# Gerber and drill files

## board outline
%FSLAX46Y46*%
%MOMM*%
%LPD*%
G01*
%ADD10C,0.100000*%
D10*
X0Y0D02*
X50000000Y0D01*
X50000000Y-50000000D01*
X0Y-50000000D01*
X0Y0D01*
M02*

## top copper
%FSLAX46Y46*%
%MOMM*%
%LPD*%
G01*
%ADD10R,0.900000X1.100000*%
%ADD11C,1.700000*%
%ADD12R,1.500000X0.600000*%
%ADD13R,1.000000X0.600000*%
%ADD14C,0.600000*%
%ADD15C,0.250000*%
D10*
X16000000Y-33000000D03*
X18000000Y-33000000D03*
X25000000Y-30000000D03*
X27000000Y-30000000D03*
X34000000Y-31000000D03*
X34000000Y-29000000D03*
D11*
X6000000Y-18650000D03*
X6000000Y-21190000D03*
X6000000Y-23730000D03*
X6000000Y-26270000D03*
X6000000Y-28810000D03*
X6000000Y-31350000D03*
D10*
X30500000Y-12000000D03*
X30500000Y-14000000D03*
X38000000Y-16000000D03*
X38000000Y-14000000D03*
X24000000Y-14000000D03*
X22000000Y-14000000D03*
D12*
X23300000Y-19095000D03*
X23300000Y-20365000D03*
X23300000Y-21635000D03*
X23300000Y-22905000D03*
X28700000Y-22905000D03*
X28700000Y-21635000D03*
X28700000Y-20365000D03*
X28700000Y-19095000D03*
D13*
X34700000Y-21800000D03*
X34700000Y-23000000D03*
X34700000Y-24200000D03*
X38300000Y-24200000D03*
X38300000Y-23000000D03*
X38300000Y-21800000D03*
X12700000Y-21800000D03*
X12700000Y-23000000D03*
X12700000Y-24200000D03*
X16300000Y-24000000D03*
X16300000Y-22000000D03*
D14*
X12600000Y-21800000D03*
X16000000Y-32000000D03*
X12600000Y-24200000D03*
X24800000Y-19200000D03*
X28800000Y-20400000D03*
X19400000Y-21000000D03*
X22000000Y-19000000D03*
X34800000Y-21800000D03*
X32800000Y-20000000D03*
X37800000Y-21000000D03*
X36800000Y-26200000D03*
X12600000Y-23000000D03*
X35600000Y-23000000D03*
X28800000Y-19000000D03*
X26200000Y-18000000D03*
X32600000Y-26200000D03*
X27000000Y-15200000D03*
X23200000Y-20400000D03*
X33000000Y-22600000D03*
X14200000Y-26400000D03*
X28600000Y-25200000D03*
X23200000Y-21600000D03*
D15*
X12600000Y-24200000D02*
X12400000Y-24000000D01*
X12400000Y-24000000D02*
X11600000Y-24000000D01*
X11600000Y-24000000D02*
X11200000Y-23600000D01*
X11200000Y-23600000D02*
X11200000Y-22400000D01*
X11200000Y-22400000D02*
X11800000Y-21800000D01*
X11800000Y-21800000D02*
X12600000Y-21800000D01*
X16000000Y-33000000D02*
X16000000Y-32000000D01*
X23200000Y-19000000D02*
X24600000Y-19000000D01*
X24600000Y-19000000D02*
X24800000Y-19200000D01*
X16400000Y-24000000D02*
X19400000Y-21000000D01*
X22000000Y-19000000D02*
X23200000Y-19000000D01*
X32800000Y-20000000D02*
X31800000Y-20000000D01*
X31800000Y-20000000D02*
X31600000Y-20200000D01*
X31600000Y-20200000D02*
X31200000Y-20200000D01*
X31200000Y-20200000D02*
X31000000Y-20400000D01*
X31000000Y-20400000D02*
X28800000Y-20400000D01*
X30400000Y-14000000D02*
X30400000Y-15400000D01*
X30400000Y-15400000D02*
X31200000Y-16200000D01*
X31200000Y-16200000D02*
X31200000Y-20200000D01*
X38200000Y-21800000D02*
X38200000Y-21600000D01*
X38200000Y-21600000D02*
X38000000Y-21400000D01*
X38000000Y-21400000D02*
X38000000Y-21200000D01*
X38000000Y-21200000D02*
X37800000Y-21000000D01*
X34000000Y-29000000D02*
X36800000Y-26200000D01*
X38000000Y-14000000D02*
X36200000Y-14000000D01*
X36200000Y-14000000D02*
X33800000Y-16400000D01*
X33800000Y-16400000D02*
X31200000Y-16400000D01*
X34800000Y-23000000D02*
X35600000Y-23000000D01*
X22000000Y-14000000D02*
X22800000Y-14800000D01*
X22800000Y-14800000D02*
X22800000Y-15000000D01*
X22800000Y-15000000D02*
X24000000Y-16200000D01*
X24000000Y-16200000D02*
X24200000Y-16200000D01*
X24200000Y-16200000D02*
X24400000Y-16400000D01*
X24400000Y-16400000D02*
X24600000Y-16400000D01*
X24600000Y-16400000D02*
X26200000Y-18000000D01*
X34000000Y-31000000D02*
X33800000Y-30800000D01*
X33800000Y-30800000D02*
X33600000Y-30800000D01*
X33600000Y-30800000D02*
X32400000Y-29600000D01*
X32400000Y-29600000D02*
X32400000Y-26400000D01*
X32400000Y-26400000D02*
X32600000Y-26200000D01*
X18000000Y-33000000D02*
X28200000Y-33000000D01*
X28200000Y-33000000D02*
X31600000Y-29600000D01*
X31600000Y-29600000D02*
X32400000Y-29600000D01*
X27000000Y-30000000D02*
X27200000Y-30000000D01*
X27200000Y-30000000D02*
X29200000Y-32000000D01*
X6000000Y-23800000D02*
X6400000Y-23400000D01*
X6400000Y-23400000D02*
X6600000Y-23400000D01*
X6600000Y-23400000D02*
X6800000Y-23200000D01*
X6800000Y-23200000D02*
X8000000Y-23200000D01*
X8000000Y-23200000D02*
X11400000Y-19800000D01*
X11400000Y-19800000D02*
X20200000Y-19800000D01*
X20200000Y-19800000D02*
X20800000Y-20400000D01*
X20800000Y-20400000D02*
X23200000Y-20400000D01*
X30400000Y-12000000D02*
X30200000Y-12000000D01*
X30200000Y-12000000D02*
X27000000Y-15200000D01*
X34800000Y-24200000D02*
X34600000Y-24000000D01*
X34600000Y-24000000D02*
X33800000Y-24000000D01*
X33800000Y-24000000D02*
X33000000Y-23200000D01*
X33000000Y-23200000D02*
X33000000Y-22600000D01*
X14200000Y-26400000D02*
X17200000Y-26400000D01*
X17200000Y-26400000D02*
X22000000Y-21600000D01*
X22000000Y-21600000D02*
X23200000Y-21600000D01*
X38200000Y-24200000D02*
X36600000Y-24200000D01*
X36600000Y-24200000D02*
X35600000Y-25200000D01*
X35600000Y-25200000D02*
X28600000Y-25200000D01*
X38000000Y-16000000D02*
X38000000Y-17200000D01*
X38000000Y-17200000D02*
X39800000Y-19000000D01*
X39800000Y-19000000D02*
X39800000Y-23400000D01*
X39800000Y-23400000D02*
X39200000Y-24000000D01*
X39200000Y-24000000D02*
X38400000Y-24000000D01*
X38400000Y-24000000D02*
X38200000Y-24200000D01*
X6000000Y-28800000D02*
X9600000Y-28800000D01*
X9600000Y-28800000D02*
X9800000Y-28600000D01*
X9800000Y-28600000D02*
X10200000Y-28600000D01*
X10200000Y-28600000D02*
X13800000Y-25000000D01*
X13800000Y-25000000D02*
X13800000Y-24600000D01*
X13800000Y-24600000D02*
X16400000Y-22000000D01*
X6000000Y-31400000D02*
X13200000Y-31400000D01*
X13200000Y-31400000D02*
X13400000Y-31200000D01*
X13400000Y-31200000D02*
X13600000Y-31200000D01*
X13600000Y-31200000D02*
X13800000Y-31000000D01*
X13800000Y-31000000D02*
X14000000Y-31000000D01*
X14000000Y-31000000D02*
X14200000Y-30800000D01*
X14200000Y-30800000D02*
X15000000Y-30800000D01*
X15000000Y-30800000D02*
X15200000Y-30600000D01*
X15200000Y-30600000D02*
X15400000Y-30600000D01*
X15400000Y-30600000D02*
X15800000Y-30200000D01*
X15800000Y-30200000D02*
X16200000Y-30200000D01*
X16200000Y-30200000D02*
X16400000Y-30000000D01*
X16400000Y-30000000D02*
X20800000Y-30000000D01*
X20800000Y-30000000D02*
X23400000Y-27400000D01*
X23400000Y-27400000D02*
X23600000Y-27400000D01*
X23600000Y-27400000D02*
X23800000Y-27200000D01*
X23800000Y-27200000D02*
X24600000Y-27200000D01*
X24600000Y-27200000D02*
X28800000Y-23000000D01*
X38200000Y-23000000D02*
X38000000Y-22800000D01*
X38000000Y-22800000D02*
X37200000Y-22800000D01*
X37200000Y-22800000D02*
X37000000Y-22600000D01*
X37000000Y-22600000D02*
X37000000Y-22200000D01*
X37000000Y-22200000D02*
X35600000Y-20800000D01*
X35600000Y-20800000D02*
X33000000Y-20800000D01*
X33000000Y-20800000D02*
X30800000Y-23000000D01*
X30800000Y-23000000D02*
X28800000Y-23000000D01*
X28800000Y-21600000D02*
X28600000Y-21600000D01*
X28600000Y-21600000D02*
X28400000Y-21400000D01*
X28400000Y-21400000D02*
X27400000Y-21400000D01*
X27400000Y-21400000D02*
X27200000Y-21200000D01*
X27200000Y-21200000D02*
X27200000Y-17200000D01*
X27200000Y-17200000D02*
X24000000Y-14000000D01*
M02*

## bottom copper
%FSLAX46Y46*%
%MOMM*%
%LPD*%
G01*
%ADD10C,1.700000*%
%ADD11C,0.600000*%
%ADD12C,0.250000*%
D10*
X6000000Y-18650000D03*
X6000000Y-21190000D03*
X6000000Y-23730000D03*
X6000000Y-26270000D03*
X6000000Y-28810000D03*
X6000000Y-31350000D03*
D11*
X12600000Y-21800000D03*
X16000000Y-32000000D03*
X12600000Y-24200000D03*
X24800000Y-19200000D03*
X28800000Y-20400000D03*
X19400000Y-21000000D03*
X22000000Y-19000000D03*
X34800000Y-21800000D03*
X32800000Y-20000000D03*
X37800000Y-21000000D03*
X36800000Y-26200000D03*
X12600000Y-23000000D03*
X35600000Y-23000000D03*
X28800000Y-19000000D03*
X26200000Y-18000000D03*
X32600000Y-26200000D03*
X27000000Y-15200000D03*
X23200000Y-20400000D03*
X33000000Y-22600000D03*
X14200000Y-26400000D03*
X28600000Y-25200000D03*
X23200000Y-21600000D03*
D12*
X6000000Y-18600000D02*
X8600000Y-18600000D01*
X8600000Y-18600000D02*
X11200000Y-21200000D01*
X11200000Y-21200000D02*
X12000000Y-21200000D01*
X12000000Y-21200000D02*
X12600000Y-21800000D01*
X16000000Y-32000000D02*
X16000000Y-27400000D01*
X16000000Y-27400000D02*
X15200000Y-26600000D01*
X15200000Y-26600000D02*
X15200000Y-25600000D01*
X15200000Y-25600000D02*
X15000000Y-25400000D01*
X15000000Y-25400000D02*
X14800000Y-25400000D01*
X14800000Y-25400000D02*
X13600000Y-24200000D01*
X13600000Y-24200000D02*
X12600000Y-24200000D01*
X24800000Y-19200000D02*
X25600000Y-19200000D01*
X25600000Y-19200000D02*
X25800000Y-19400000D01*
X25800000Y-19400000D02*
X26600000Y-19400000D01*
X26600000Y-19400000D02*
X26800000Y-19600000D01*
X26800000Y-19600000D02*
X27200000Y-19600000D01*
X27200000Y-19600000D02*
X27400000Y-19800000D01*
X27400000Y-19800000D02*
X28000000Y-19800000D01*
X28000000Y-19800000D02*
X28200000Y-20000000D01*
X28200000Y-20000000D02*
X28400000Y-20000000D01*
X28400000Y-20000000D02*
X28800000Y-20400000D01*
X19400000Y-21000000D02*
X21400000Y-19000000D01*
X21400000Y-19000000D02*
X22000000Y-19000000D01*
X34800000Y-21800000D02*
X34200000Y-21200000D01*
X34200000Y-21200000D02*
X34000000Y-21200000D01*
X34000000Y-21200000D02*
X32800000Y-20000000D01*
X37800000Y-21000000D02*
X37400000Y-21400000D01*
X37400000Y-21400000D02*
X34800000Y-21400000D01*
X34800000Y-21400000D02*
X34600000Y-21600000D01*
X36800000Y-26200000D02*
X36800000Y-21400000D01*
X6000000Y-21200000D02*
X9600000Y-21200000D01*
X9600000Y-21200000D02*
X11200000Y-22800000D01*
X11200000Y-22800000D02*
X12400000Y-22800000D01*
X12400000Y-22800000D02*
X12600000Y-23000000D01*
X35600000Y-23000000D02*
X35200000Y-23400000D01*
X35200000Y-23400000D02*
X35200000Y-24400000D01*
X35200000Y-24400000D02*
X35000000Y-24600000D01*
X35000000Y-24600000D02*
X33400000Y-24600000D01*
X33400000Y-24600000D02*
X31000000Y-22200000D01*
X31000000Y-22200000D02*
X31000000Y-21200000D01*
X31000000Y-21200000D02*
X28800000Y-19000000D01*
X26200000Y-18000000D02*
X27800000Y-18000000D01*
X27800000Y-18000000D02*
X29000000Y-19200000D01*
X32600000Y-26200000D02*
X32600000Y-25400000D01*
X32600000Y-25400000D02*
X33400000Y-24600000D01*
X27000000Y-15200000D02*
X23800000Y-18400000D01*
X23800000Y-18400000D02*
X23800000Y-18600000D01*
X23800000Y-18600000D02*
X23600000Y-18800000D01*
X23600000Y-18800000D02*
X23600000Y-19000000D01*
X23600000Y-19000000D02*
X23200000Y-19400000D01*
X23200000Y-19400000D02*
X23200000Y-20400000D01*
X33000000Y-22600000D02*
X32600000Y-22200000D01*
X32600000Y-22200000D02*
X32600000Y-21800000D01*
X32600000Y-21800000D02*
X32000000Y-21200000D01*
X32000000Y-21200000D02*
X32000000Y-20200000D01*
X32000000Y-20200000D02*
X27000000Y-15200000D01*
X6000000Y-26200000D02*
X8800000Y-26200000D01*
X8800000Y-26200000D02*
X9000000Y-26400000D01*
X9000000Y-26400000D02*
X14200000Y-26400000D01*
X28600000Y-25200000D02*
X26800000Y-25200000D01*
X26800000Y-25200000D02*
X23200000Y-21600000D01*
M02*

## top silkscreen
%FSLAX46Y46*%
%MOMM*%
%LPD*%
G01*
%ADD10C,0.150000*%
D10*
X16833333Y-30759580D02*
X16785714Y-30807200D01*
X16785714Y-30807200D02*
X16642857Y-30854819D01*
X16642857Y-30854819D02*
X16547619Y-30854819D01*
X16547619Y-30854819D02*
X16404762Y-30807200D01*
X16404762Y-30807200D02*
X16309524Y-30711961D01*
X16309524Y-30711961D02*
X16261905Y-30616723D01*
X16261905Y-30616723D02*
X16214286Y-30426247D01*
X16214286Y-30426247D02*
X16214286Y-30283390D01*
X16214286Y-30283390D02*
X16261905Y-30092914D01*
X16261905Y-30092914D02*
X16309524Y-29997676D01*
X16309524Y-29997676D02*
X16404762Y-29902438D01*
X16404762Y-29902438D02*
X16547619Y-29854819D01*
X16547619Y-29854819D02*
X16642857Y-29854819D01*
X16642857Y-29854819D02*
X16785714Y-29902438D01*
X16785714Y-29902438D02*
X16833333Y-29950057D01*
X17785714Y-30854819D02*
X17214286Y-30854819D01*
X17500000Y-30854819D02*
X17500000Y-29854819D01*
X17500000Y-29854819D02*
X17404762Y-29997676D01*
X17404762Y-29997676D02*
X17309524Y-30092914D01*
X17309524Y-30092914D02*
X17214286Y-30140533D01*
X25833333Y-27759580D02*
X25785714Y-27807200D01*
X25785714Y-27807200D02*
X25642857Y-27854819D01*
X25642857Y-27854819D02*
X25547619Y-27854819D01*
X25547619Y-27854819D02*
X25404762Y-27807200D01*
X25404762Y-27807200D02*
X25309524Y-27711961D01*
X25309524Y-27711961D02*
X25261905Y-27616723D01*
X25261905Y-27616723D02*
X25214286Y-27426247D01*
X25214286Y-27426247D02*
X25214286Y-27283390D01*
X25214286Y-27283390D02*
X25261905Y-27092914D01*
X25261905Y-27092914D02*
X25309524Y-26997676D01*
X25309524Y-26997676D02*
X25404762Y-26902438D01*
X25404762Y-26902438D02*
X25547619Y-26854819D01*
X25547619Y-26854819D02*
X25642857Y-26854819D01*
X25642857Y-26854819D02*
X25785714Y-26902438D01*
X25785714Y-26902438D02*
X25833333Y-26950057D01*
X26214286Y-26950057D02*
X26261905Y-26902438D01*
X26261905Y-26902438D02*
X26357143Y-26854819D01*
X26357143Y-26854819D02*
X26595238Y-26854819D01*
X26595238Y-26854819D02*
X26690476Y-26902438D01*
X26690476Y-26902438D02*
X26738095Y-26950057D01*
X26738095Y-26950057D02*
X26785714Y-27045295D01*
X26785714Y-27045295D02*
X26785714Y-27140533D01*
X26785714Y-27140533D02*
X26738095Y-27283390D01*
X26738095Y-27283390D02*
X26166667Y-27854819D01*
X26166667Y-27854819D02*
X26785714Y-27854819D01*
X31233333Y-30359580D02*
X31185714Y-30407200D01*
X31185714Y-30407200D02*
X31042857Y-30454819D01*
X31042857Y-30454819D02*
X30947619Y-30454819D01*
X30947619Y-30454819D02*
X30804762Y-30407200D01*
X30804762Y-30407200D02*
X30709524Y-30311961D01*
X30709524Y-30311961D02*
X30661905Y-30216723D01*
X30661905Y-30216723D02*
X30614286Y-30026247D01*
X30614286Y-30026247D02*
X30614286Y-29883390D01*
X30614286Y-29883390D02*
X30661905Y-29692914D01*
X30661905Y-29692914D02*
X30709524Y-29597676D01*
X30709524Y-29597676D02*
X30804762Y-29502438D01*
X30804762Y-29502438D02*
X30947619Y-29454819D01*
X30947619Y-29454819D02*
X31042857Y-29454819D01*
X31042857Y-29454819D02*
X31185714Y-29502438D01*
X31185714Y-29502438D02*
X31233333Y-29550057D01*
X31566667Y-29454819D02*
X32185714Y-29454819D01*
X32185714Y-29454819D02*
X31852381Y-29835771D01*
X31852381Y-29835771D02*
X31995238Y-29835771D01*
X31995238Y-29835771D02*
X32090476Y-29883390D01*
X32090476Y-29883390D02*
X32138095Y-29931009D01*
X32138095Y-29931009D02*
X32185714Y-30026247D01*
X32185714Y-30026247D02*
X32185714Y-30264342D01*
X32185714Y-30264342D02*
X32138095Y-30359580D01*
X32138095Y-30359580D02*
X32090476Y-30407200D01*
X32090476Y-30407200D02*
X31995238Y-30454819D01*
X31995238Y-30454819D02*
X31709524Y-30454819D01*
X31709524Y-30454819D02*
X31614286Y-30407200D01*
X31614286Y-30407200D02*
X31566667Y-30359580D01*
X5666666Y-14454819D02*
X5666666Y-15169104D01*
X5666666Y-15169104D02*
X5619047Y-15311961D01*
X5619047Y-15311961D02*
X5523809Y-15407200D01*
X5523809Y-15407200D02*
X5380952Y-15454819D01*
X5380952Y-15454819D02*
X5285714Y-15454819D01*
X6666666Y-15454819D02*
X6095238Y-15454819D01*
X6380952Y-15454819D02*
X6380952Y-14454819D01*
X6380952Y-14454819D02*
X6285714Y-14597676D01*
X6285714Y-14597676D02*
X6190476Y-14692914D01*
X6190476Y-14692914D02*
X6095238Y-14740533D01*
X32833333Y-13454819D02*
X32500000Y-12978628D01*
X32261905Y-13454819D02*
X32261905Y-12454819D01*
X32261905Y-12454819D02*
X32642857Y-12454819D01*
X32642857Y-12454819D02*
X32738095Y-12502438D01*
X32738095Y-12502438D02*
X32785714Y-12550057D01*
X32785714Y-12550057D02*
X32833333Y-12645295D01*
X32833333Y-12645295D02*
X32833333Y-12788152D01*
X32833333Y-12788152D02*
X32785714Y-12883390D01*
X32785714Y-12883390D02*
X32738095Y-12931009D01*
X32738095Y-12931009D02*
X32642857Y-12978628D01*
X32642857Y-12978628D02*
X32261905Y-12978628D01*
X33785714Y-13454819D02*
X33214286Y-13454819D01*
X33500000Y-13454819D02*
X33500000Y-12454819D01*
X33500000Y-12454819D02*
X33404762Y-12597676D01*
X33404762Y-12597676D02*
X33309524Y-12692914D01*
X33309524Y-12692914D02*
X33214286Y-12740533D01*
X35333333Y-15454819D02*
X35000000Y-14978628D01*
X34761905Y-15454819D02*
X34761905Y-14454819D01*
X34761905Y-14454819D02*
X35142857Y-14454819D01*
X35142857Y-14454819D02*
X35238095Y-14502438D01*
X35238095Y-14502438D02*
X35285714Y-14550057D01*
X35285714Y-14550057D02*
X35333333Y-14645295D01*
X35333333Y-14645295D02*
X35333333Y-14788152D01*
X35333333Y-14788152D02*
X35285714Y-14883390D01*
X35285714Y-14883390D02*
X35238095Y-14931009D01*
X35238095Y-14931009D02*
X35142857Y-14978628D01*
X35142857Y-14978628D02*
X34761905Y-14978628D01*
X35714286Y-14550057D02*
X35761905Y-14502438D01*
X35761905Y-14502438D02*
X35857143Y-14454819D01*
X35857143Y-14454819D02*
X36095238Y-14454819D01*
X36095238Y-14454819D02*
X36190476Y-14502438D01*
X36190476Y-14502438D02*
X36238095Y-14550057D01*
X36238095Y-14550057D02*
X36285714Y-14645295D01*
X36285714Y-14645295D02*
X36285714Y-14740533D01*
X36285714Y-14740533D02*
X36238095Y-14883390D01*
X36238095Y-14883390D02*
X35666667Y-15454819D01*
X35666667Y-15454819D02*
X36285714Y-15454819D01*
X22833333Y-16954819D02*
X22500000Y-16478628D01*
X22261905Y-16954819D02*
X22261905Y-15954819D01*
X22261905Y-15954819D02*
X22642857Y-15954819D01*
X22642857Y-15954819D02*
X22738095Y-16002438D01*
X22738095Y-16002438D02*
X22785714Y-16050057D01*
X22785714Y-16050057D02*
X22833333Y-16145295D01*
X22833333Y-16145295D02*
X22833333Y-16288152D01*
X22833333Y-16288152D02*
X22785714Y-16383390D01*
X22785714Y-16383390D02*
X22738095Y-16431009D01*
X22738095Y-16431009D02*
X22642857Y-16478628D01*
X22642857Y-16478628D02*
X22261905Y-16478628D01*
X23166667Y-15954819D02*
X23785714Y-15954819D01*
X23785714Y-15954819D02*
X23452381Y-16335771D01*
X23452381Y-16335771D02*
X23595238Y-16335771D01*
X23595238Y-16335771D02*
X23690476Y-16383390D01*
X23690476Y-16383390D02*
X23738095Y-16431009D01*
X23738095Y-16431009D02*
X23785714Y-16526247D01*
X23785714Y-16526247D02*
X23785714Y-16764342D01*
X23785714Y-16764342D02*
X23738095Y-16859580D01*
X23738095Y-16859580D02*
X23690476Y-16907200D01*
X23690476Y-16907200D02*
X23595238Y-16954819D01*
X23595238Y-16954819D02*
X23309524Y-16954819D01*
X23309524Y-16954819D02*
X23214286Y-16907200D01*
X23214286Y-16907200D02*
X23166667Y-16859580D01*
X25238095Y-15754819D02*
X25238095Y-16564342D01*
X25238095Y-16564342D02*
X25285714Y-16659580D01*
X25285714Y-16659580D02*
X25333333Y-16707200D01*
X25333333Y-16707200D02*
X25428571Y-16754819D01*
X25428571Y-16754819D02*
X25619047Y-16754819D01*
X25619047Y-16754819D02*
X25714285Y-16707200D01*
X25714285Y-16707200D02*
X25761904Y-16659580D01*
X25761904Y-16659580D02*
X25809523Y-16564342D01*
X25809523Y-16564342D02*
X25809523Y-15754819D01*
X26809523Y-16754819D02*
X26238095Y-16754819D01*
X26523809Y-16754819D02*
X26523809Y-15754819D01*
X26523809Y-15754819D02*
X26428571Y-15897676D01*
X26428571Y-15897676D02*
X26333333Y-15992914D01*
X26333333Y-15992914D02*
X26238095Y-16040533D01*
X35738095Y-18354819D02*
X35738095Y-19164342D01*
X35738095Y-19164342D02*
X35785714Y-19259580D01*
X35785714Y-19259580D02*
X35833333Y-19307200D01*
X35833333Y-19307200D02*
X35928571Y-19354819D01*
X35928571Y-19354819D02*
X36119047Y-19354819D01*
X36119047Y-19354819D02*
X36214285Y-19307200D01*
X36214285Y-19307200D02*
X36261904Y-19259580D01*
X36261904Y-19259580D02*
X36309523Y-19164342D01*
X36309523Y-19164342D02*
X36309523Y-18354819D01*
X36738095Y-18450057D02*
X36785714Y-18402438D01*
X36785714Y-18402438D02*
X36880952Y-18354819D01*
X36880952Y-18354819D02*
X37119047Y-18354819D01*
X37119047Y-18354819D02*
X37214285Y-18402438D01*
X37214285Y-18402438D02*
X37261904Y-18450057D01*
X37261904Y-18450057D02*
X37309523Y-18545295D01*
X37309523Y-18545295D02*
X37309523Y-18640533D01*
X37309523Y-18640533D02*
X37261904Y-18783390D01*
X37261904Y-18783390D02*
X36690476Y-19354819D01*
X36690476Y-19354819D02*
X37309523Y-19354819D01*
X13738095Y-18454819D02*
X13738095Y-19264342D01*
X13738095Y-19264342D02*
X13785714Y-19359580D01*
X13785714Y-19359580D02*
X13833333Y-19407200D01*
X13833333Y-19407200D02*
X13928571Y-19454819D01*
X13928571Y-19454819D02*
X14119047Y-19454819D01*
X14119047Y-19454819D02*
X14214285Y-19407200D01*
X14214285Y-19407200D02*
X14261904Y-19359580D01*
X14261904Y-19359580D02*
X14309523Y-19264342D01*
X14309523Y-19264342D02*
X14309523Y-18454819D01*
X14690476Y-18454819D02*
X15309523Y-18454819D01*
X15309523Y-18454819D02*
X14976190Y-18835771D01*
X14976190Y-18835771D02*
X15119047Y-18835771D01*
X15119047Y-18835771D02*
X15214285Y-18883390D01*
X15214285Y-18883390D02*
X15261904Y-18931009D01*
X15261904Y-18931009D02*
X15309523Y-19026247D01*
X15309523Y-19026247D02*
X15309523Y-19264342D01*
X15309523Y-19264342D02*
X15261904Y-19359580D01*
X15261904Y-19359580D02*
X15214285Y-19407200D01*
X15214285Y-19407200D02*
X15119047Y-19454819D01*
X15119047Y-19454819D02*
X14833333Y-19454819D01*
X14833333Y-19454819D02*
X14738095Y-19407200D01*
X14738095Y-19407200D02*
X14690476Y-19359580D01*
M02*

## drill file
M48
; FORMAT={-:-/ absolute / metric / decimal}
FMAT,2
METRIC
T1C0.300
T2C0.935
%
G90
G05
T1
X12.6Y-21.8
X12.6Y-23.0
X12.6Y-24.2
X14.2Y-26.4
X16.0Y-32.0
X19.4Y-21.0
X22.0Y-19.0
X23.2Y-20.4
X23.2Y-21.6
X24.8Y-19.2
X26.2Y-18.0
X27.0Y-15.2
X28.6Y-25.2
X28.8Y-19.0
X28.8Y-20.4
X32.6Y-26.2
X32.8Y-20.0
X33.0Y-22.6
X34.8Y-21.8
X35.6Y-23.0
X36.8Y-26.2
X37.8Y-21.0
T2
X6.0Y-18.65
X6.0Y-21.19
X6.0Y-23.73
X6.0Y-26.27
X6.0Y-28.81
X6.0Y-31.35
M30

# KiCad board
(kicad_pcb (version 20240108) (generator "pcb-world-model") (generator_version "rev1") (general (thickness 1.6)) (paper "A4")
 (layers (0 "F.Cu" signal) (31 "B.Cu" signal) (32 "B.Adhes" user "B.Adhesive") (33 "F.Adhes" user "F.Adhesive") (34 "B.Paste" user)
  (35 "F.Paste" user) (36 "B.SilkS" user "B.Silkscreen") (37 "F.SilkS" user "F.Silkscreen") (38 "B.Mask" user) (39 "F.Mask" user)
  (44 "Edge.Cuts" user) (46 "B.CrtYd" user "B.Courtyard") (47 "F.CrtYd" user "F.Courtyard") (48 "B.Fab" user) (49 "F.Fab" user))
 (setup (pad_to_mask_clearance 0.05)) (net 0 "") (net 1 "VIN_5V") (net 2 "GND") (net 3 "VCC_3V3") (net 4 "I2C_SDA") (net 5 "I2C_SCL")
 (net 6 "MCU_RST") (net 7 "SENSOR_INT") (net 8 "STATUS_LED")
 (gr_rect (start 0.0 0.0) (end 50.0000 50.0000) (stroke (width 0.1) (type default)) (fill none) (layer "Edge.Cuts"))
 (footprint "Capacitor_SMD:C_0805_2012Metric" (layer "F.Cu") (at 17.0000 33.0000 0)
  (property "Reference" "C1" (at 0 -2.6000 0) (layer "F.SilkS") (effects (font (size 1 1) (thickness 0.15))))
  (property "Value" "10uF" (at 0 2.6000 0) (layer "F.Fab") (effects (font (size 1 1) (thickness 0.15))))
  (pad "1" smd rect (at -1.0000 0.0000) (size 0.9000 1.1000) (layers "F.Cu" "F.Paste" "F.Mask") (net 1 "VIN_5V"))
  (pad "2" smd rect (at 1.0000 0.0000) (size 0.9000 1.1000) (layers "F.Cu" "F.Paste" "F.Mask") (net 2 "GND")))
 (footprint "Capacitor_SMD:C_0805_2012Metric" (layer "F.Cu") (at 26.0000 30.0000 0)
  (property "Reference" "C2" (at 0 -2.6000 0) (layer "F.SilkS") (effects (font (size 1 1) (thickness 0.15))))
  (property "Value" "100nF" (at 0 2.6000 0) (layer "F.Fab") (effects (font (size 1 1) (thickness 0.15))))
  (pad "1" smd rect (at -1.0000 0.0000) (size 0.9000 1.1000) (layers "F.Cu" "F.Paste" "F.Mask") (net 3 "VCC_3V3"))
  (pad "2" smd rect (at 1.0000 0.0000) (size 0.9000 1.1000) (layers "F.Cu" "F.Paste" "F.Mask") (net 2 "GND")))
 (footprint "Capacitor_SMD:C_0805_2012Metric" (layer "F.Cu") (at 34.0000 30.0000 90)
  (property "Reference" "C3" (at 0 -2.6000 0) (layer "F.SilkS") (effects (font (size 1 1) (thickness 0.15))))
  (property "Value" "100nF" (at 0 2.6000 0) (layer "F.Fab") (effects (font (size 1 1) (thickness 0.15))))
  (pad "1" smd rect (at -1.0000 0.0000) (size 0.9000 1.1000) (layers "F.Cu" "F.Paste" "F.Mask") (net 3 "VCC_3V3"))
  (pad "2" smd rect (at 1.0000 0.0000) (size 0.9000 1.1000) (layers "F.Cu" "F.Paste" "F.Mask") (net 2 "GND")))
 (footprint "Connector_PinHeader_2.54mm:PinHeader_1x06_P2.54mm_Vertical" (layer "F.Cu") (at 6.0000 25.0000 0) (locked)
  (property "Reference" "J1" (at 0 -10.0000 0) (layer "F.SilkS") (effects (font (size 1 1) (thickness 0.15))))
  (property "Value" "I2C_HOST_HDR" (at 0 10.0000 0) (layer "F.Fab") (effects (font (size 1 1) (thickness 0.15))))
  (pad "1" thru_hole circle (at 0.0000 -6.3500) (size 1.7000 1.7000) (drill 0.9350) (layers "*.Cu" "*.Mask") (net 1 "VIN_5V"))
  (pad "2" thru_hole circle (at 0.0000 -3.8100) (size 1.7000 1.7000) (drill 0.9350) (layers "*.Cu" "*.Mask") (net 2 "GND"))
  (pad "3" thru_hole circle (at 0.0000 -1.2700) (size 1.7000 1.7000) (drill 0.9350) (layers "*.Cu" "*.Mask") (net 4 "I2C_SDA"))
  (pad "4" thru_hole circle (at 0.0000 1.2700) (size 1.7000 1.7000) (drill 0.9350) (layers "*.Cu" "*.Mask") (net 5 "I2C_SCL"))
  (pad "5" thru_hole circle (at 0.0000 3.8100) (size 1.7000 1.7000) (drill 0.9350) (layers "*.Cu" "*.Mask") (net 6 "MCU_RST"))
  (pad "6" thru_hole circle (at 0.0000 6.3500) (size 1.7000 1.7000) (drill 0.9350) (layers "*.Cu" "*.Mask") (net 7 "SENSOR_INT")))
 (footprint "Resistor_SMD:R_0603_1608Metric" (layer "F.Cu") (at 30.5000 13.0000 270)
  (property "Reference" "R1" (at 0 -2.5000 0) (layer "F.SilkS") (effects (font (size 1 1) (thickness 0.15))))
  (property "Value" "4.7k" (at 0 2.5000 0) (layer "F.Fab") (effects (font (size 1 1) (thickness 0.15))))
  (pad "1" smd rect (at -1.0000 0.0000) (size 0.9000 1.1000) (layers "F.Cu" "F.Paste" "F.Mask") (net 3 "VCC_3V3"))
  (pad "2" smd rect (at 1.0000 0.0000) (size 0.9000 1.1000) (layers "F.Cu" "F.Paste" "F.Mask") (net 4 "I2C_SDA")))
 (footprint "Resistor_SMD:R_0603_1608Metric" (layer "F.Cu") (at 38.0000 15.0000 90)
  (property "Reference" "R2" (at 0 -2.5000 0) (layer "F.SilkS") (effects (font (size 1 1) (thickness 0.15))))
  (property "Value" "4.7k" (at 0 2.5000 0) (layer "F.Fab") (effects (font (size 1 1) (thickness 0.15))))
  (pad "1" smd rect (at -1.0000 0.0000) (size 0.9000 1.1000) (layers "F.Cu" "F.Paste" "F.Mask") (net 3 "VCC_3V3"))
  (pad "2" smd rect (at 1.0000 0.0000) (size 0.9000 1.1000) (layers "F.Cu" "F.Paste" "F.Mask") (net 5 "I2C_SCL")))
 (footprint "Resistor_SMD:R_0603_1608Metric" (layer "F.Cu") (at 23.0000 14.0000 180)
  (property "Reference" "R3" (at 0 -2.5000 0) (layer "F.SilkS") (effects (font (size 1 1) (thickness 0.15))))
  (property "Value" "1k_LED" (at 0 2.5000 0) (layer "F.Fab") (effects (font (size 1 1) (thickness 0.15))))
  (pad "1" smd rect (at -1.0000 0.0000) (size 0.9000 1.1000) (layers "F.Cu" "F.Paste" "F.Mask") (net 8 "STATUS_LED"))
  (pad "2" smd rect (at 1.0000 0.0000) (size 0.9000 1.1000) (layers "F.Cu" "F.Paste" "F.Mask") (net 2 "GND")))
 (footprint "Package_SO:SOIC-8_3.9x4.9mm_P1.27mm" (layer "F.Cu") (at 26.0000 21.0000 0)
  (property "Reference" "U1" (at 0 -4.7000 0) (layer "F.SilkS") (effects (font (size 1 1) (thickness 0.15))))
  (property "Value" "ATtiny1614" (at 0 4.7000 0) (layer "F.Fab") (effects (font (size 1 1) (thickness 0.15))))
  (pad "1" smd rect (at -2.7000 -1.9050) (size 1.5000 0.6000) (layers "F.Cu" "F.Paste" "F.Mask") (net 3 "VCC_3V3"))
  (pad "2" smd rect (at -2.7000 -0.6350) (size 1.5000 0.6000) (layers "F.Cu" "F.Paste" "F.Mask") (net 4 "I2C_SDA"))
  (pad "3" smd rect (at -2.7000 0.6350) (size 1.5000 0.6000) (layers "F.Cu" "F.Paste" "F.Mask") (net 5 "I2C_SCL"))
  (pad "4" smd rect (at -2.7000 1.9050) (size 1.5000 0.6000) (layers "F.Cu" "F.Paste" "F.Mask") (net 6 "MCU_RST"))
  (pad "5" smd rect (at 2.7000 1.9050) (size 1.5000 0.6000) (layers "F.Cu" "F.Paste" "F.Mask") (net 7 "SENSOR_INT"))
  (pad "6" smd rect (at 2.7000 0.6350) (size 1.5000 0.6000) (layers "F.Cu" "F.Paste" "F.Mask") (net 8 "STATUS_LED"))
  (pad "7" smd rect (at 2.7000 -0.6350) (size 1.5000 0.6000) (layers "F.Cu" "F.Paste" "F.Mask") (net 3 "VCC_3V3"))
  (pad "8" smd rect (at 2.7000 -1.9050) (size 1.5000 0.6000) (layers "F.Cu" "F.Paste" "F.Mask") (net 2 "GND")))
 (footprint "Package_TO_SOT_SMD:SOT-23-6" (layer "F.Cu") (at 36.5000 23.0000 0)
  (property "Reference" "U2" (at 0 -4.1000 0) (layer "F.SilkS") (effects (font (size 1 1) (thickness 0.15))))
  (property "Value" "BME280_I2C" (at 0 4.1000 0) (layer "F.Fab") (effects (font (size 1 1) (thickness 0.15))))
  (pad "1" smd rect (at -1.8000 -1.2000) (size 1.0000 0.6000) (layers "F.Cu" "F.Paste" "F.Mask") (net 3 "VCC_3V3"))
  (pad "2" smd rect (at -1.8000 0.0000) (size 1.0000 0.6000) (layers "F.Cu" "F.Paste" "F.Mask") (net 2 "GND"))
  (pad "3" smd rect (at -1.8000 1.2000) (size 1.0000 0.6000) (layers "F.Cu" "F.Paste" "F.Mask") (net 4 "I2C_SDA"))
  (pad "4" smd rect (at 1.8000 1.2000) (size 1.0000 0.6000) (layers "F.Cu" "F.Paste" "F.Mask") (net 5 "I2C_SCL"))
  (pad "5" smd rect (at 1.8000 0.0000) (size 1.0000 0.6000) (layers "F.Cu" "F.Paste" "F.Mask") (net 7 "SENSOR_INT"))
  (pad "6" smd rect (at 1.8000 -1.2000) (size 1.0000 0.6000) (layers "F.Cu" "F.Paste" "F.Mask") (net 3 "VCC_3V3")))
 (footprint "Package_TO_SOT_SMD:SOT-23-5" (layer "F.Cu") (at 14.5000 23.0000 0)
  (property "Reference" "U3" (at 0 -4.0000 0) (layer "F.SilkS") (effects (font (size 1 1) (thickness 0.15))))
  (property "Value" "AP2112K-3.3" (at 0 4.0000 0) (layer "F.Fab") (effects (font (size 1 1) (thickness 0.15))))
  (pad "1" smd rect (at -1.8000 -1.2000) (size 1.0000 0.6000) (layers "F.Cu" "F.Paste" "F.Mask") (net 1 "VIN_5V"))
  (pad "2" smd rect (at -1.8000 0.0000) (size 1.0000 0.6000) (layers "F.Cu" "F.Paste" "F.Mask") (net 2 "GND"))
  (pad "3" smd rect (at -1.8000 1.2000) (size 1.0000 0.6000) (layers "F.Cu" "F.Paste" "F.Mask") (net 1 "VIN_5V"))
  (pad "4" smd rect (at 1.8000 1.0000) (size 1.0000 0.6000) (layers "F.Cu" "F.Paste" "F.Mask") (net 3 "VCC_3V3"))
  (pad "5" smd rect (at 1.8000 -1.0000) (size 1.0000 0.6000) (layers "F.Cu" "F.Paste" "F.Mask") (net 6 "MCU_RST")))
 (segment (start 6.0000 18.6000) (end 8.6000 18.6000) (width 0.2500) (layer "B.Cu") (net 1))
 (segment (start 8.6000 18.6000) (end 11.2000 21.2000) (width 0.2500) (layer "B.Cu") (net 1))
 (segment (start 11.2000 21.2000) (end 12.0000 21.2000) (width 0.2500) (layer "B.Cu") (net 1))
 (segment (start 12.0000 21.2000) (end 12.6000 21.8000) (width 0.2500) (layer "B.Cu") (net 1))
 (segment (start 12.6000 24.2000) (end 12.4000 24.0000) (width 0.2500) (layer "F.Cu") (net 1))
 (segment (start 12.4000 24.0000) (end 11.6000 24.0000) (width 0.2500) (layer "F.Cu") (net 1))
 (segment (start 11.6000 24.0000) (end 11.2000 23.6000) (width 0.2500) (layer "F.Cu") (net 1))
 (segment (start 11.2000 23.6000) (end 11.2000 22.4000) (width 0.2500) (layer "F.Cu") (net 1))
 (segment (start 11.2000 22.4000) (end 11.8000 21.8000) (width 0.2500) (layer "F.Cu") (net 1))
 (segment (start 11.8000 21.8000) (end 12.6000 21.8000) (width 0.2500) (layer "F.Cu") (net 1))
 (segment (start 16.0000 33.0000) (end 16.0000 32.0000) (width 0.2500) (layer "F.Cu") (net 1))
 (segment (start 16.0000 32.0000) (end 16.0000 27.4000) (width 0.2500) (layer "B.Cu") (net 1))
 (segment (start 16.0000 27.4000) (end 15.2000 26.6000) (width 0.2500) (layer "B.Cu") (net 1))
 (segment (start 15.2000 26.6000) (end 15.2000 25.6000) (width 0.2500) (layer "B.Cu") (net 1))
 (segment (start 15.2000 25.6000) (end 15.0000 25.4000) (width 0.2500) (layer "B.Cu") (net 1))
 (segment (start 15.0000 25.4000) (end 14.8000 25.4000) (width 0.2500) (layer "B.Cu") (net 1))
 (segment (start 14.8000 25.4000) (end 13.6000 24.2000) (width 0.2500) (layer "B.Cu") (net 1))
 (segment (start 13.6000 24.2000) (end 12.6000 24.2000) (width 0.2500) (layer "B.Cu") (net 1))
 (segment (start 23.2000 19.0000) (end 24.6000 19.0000) (width 0.2500) (layer "F.Cu") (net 3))
 (segment (start 24.6000 19.0000) (end 24.8000 19.2000) (width 0.2500) (layer "F.Cu") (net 3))
 (segment (start 24.8000 19.2000) (end 25.6000 19.2000) (width 0.2500) (layer "B.Cu") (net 3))
 (segment (start 25.6000 19.2000) (end 25.8000 19.4000) (width 0.2500) (layer "B.Cu") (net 3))
 (segment (start 25.8000 19.4000) (end 26.6000 19.4000) (width 0.2500) (layer "B.Cu") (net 3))
 (segment (start 26.6000 19.4000) (end 26.8000 19.6000) (width 0.2500) (layer "B.Cu") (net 3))
 (segment (start 26.8000 19.6000) (end 27.2000 19.6000) (width 0.2500) (layer "B.Cu") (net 3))
 (segment (start 27.2000 19.6000) (end 27.4000 19.8000) (width 0.2500) (layer "B.Cu") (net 3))
 (segment (start 27.4000 19.8000) (end 28.0000 19.8000) (width 0.2500) (layer "B.Cu") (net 3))
 (segment (start 28.0000 19.8000) (end 28.2000 20.0000) (width 0.2500) (layer "B.Cu") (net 3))
 (segment (start 28.2000 20.0000) (end 28.4000 20.0000) (width 0.2500) (layer "B.Cu") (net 3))
 (segment (start 28.4000 20.0000) (end 28.8000 20.4000) (width 0.2500) (layer "B.Cu") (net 3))
 (segment (start 16.4000 24.0000) (end 19.4000 21.0000) (width 0.2500) (layer "F.Cu") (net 3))
 (segment (start 19.4000 21.0000) (end 21.4000 19.0000) (width 0.2500) (layer "B.Cu") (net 3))
 (segment (start 21.4000 19.0000) (end 22.0000 19.0000) (width 0.2500) (layer "B.Cu") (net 3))
 (segment (start 22.0000 19.0000) (end 23.2000 19.0000) (width 0.2500) (layer "F.Cu") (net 3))
 (segment (start 34.8000 21.8000) (end 34.2000 21.2000) (width 0.2500) (layer "B.Cu") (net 3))
 (segment (start 34.2000 21.2000) (end 34.0000 21.2000) (width 0.2500) (layer "B.Cu") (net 3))
 (segment (start 34.0000 21.2000) (end 32.8000 20.0000) (width 0.2500) (layer "B.Cu") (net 3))
 (segment (start 32.8000 20.0000) (end 31.8000 20.0000) (width 0.2500) (layer "F.Cu") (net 3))
 (segment (start 31.8000 20.0000) (end 31.6000 20.2000) (width 0.2500) (layer "F.Cu") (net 3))
 (segment (start 31.6000 20.2000) (end 31.2000 20.2000) (width 0.2500) (layer "F.Cu") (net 3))
 (segment (start 31.2000 20.2000) (end 31.0000 20.4000) (width 0.2500) (layer "F.Cu") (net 3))
 (segment (start 31.0000 20.4000) (end 28.8000 20.4000) (width 0.2500) (layer "F.Cu") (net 3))
 (segment (start 30.4000 14.0000) (end 30.4000 15.4000) (width 0.2500) (layer "F.Cu") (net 3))
 (segment (start 30.4000 15.4000) (end 31.2000 16.2000) (width 0.2500) (layer "F.Cu") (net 3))
 (segment (start 31.2000 16.2000) (end 31.2000 20.2000) (width 0.2500) (layer "F.Cu") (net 3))
 (segment (start 38.2000 21.8000) (end 38.2000 21.6000) (width 0.2500) (layer "F.Cu") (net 3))
 (segment (start 38.2000 21.6000) (end 38.0000 21.4000) (width 0.2500) (layer "F.Cu") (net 3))
 (segment (start 38.0000 21.4000) (end 38.0000 21.2000) (width 0.2500) (layer "F.Cu") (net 3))
 (segment (start 38.0000 21.2000) (end 37.8000 21.0000) (width 0.2500) (layer "F.Cu") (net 3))
 (segment (start 37.8000 21.0000) (end 37.4000 21.4000) (width 0.2500) (layer "B.Cu") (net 3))
 (segment (start 37.4000 21.4000) (end 34.8000 21.4000) (width 0.2500) (layer "B.Cu") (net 3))
 (segment (start 34.8000 21.4000) (end 34.6000 21.6000) (width 0.2500) (layer "B.Cu") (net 3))
 (segment (start 34.0000 29.0000) (end 36.8000 26.2000) (width 0.2500) (layer "F.Cu") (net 3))
 (segment (start 36.8000 26.2000) (end 36.8000 21.4000) (width 0.2500) (layer "B.Cu") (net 3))
 (segment (start 38.0000 14.0000) (end 36.2000 14.0000) (width 0.2500) (layer "F.Cu") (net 3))
 (segment (start 36.2000 14.0000) (end 33.8000 16.4000) (width 0.2500) (layer "F.Cu") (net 3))
 (segment (start 33.8000 16.4000) (end 31.2000 16.4000) (width 0.2500) (layer "F.Cu") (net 3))
 (segment (start 6.0000 21.2000) (end 9.6000 21.2000) (width 0.2500) (layer "B.Cu") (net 2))
 (segment (start 9.6000 21.2000) (end 11.2000 22.8000) (width 0.2500) (layer "B.Cu") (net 2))
 (segment (start 11.2000 22.8000) (end 12.4000 22.8000) (width 0.2500) (layer "B.Cu") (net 2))
 (segment (start 12.4000 22.8000) (end 12.6000 23.0000) (width 0.2500) (layer "B.Cu") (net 2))
 (segment (start 34.8000 23.0000) (end 35.6000 23.0000) (width 0.2500) (layer "F.Cu") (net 2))
 (segment (start 35.6000 23.0000) (end 35.2000 23.4000) (width 0.2500) (layer "B.Cu") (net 2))
 (segment (start 35.2000 23.4000) (end 35.2000 24.4000) (width 0.2500) (layer "B.Cu") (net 2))
 (segment (start 35.2000 24.4000) (end 35.0000 24.6000) (width 0.2500) (layer "B.Cu") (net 2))
 (segment (start 35.0000 24.6000) (end 33.4000 24.6000) (width 0.2500) (layer "B.Cu") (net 2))
 (segment (start 33.4000 24.6000) (end 31.0000 22.2000) (width 0.2500) (layer "B.Cu") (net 2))
 (segment (start 31.0000 22.2000) (end 31.0000 21.2000) (width 0.2500) (layer "B.Cu") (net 2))
 (segment (start 31.0000 21.2000) (end 28.8000 19.0000) (width 0.2500) (layer "B.Cu") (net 2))
 (segment (start 22.0000 14.0000) (end 22.8000 14.8000) (width 0.2500) (layer "F.Cu") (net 2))
 (segment (start 22.8000 14.8000) (end 22.8000 15.0000) (width 0.2500) (layer "F.Cu") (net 2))
 (segment (start 22.8000 15.0000) (end 24.0000 16.2000) (width 0.2500) (layer "F.Cu") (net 2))
 (segment (start 24.0000 16.2000) (end 24.2000 16.2000) (width 0.2500) (layer "F.Cu") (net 2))
 (segment (start 24.2000 16.2000) (end 24.4000 16.4000) (width 0.2500) (layer "F.Cu") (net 2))
 (segment (start 24.4000 16.4000) (end 24.6000 16.4000) (width 0.2500) (layer "F.Cu") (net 2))
 (segment (start 24.6000 16.4000) (end 26.2000 18.0000) (width 0.2500) (layer "F.Cu") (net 2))
 (segment (start 26.2000 18.0000) (end 27.8000 18.0000) (width 0.2500) (layer "B.Cu") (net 2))
 (segment (start 27.8000 18.0000) (end 29.0000 19.2000) (width 0.2500) (layer "B.Cu") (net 2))
 (segment (start 34.0000 31.0000) (end 33.8000 30.8000) (width 0.2500) (layer "F.Cu") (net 2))
 (segment (start 33.8000 30.8000) (end 33.6000 30.8000) (width 0.2500) (layer "F.Cu") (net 2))
 (segment (start 33.6000 30.8000) (end 32.4000 29.6000) (width 0.2500) (layer "F.Cu") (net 2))
 (segment (start 32.4000 29.6000) (end 32.4000 26.4000) (width 0.2500) (layer "F.Cu") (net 2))
 (segment (start 32.4000 26.4000) (end 32.6000 26.2000) (width 0.2500) (layer "F.Cu") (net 2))
 (segment (start 32.6000 26.2000) (end 32.6000 25.4000) (width 0.2500) (layer "B.Cu") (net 2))
 (segment (start 32.6000 25.4000) (end 33.4000 24.6000) (width 0.2500) (layer "B.Cu") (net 2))
 (segment (start 18.0000 33.0000) (end 28.2000 33.0000) (width 0.2500) (layer "F.Cu") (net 2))
 (segment (start 28.2000 33.0000) (end 31.6000 29.6000) (width 0.2500) (layer "F.Cu") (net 2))
 (segment (start 31.6000 29.6000) (end 32.4000 29.6000) (width 0.2500) (layer "F.Cu") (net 2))
 (segment (start 27.0000 30.0000) (end 27.2000 30.0000) (width 0.2500) (layer "F.Cu") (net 2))
 (segment (start 27.2000 30.0000) (end 29.2000 32.0000) (width 0.2500) (layer "F.Cu") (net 2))
 (segment (start 6.0000 23.8000) (end 6.4000 23.4000) (width 0.2500) (layer "F.Cu") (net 4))
 (segment (start 6.4000 23.4000) (end 6.6000 23.4000) (width 0.2500) (layer "F.Cu") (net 4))
 (segment (start 6.6000 23.4000) (end 6.8000 23.2000) (width 0.2500) (layer "F.Cu") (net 4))
 (segment (start 6.8000 23.2000) (end 8.0000 23.2000) (width 0.2500) (layer "F.Cu") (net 4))
 (segment (start 8.0000 23.2000) (end 11.4000 19.8000) (width 0.2500) (layer "F.Cu") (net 4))
 (segment (start 11.4000 19.8000) (end 20.2000 19.8000) (width 0.2500) (layer "F.Cu") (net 4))
 (segment (start 20.2000 19.8000) (end 20.8000 20.4000) (width 0.2500) (layer "F.Cu") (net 4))
 (segment (start 20.8000 20.4000) (end 23.2000 20.4000) (width 0.2500) (layer "F.Cu") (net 4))
 (segment (start 30.4000 12.0000) (end 30.2000 12.0000) (width 0.2500) (layer "F.Cu") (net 4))
 (segment (start 30.2000 12.0000) (end 27.0000 15.2000) (width 0.2500) (layer "F.Cu") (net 4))
 (segment (start 27.0000 15.2000) (end 23.8000 18.4000) (width 0.2500) (layer "B.Cu") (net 4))
 (segment (start 23.8000 18.4000) (end 23.8000 18.6000) (width 0.2500) (layer "B.Cu") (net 4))
 (segment (start 23.8000 18.6000) (end 23.6000 18.8000) (width 0.2500) (layer "B.Cu") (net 4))
 (segment (start 23.6000 18.8000) (end 23.6000 19.0000) (width 0.2500) (layer "B.Cu") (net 4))
 (segment (start 23.6000 19.0000) (end 23.2000 19.4000) (width 0.2500) (layer "B.Cu") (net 4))
 (segment (start 23.2000 19.4000) (end 23.2000 20.4000) (width 0.2500) (layer "B.Cu") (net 4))
 (segment (start 34.8000 24.2000) (end 34.6000 24.0000) (width 0.2500) (layer "F.Cu") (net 4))
 (segment (start 34.6000 24.0000) (end 33.8000 24.0000) (width 0.2500) (layer "F.Cu") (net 4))
 (segment (start 33.8000 24.0000) (end 33.0000 23.2000) (width 0.2500) (layer "F.Cu") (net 4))
 (segment (start 33.0000 23.2000) (end 33.0000 22.6000) (width 0.2500) (layer "F.Cu") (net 4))
 (segment (start 33.0000 22.6000) (end 32.6000 22.2000) (width 0.2500) (layer "B.Cu") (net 4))
 (segment (start 32.6000 22.2000) (end 32.6000 21.8000) (width 0.2500) (layer "B.Cu") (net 4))
 (segment (start 32.6000 21.8000) (end 32.0000 21.2000) (width 0.2500) (layer "B.Cu") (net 4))
 (segment (start 32.0000 21.2000) (end 32.0000 20.2000) (width 0.2500) (layer "B.Cu") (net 4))
 (segment (start 32.0000 20.2000) (end 27.0000 15.2000) (width 0.2500) (layer "B.Cu") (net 4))
 (segment (start 6.0000 26.2000) (end 8.8000 26.2000) (width 0.2500) (layer "B.Cu") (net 5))
 (segment (start 8.8000 26.2000) (end 9.0000 26.4000) (width 0.2500) (layer "B.Cu") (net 5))
 (segment (start 9.0000 26.4000) (end 14.2000 26.4000) (width 0.2500) (layer "B.Cu") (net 5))
 (segment (start 14.2000 26.4000) (end 17.2000 26.4000) (width 0.2500) (layer "F.Cu") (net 5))
 (segment (start 17.2000 26.4000) (end 22.0000 21.6000) (width 0.2500) (layer "F.Cu") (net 5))
 (segment (start 22.0000 21.6000) (end 23.2000 21.6000) (width 0.2500) (layer "F.Cu") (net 5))
 (segment (start 38.2000 24.2000) (end 36.6000 24.2000) (width 0.2500) (layer "F.Cu") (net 5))
 (segment (start 36.6000 24.2000) (end 35.6000 25.2000) (width 0.2500) (layer "F.Cu") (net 5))
 (segment (start 35.6000 25.2000) (end 28.6000 25.2000) (width 0.2500) (layer "F.Cu") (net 5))
 (segment (start 28.6000 25.2000) (end 26.8000 25.2000) (width 0.2500) (layer "B.Cu") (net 5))
 (segment (start 26.8000 25.2000) (end 23.2000 21.6000) (width 0.2500) (layer "B.Cu") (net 5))
 (segment (start 38.0000 16.0000) (end 38.0000 17.2000) (width 0.2500) (layer "F.Cu") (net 5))
 (segment (start 38.0000 17.2000) (end 39.8000 19.0000) (width 0.2500) (layer "F.Cu") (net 5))
 (segment (start 39.8000 19.0000) (end 39.8000 23.4000) (width 0.2500) (layer "F.Cu") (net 5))
 (segment (start 39.8000 23.4000) (end 39.2000 24.0000) (width 0.2500) (layer "F.Cu") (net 5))
 (segment (start 39.2000 24.0000) (end 38.4000 24.0000) (width 0.2500) (layer "F.Cu") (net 5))
 (segment (start 38.4000 24.0000) (end 38.2000 24.2000) (width 0.2500) (layer "F.Cu") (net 5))
 (segment (start 6.0000 28.8000) (end 9.6000 28.8000) (width 0.2500) (layer "F.Cu") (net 6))
 (segment (start 9.6000 28.8000) (end 9.8000 28.6000) (width 0.2500) (layer "F.Cu") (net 6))
 (segment (start 9.8000 28.6000) (end 10.2000 28.6000) (width 0.2500) (layer "F.Cu") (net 6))
 (segment (start 10.2000 28.6000) (end 13.8000 25.0000) (width 0.2500) (layer "F.Cu") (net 6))
 (segment (start 13.8000 25.0000) (end 13.8000 24.6000) (width 0.2500) (layer "F.Cu") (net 6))
 (segment (start 13.8000 24.6000) (end 16.4000 22.0000) (width 0.2500) (layer "F.Cu") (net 6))
 (segment (start 6.0000 31.4000) (end 13.2000 31.4000) (width 0.2500) (layer "F.Cu") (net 7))
 (segment (start 13.2000 31.4000) (end 13.4000 31.2000) (width 0.2500) (layer "F.Cu") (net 7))
 (segment (start 13.4000 31.2000) (end 13.6000 31.2000) (width 0.2500) (layer "F.Cu") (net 7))
 (segment (start 13.6000 31.2000) (end 13.8000 31.0000) (width 0.2500) (layer "F.Cu") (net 7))
 (segment (start 13.8000 31.0000) (end 14.0000 31.0000) (width 0.2500) (layer "F.Cu") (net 7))
 (segment (start 14.0000 31.0000) (end 14.2000 30.8000) (width 0.2500) (layer "F.Cu") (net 7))
 (segment (start 14.2000 30.8000) (end 15.0000 30.8000) (width 0.2500) (layer "F.Cu") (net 7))
 (segment (start 15.0000 30.8000) (end 15.2000 30.6000) (width 0.2500) (layer "F.Cu") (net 7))
 (segment (start 15.2000 30.6000) (end 15.4000 30.6000) (width 0.2500) (layer "F.Cu") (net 7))
 (segment (start 15.4000 30.6000) (end 15.8000 30.2000) (width 0.2500) (layer "F.Cu") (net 7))
 (segment (start 15.8000 30.2000) (end 16.2000 30.2000) (width 0.2500) (layer "F.Cu") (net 7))
 (segment (start 16.2000 30.2000) (end 16.4000 30.0000) (width 0.2500) (layer "F.Cu") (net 7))
 (segment (start 16.4000 30.0000) (end 20.8000 30.0000) (width 0.2500) (layer "F.Cu") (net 7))
 (segment (start 20.8000 30.0000) (end 23.4000 27.4000) (width 0.2500) (layer "F.Cu") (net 7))
 (segment (start 23.4000 27.4000) (end 23.6000 27.4000) (width 0.2500) (layer "F.Cu") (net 7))
 (segment (start 23.6000 27.4000) (end 23.8000 27.2000) (width 0.2500) (layer "F.Cu") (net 7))
 (segment (start 23.8000 27.2000) (end 24.6000 27.2000) (width 0.2500) (layer "F.Cu") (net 7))
 (segment (start 24.6000 27.2000) (end 28.8000 23.0000) (width 0.2500) (layer "F.Cu") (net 7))
 (segment (start 38.2000 23.0000) (end 38.0000 22.8000) (width 0.2500) (layer "F.Cu") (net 7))
 (segment (start 38.0000 22.8000) (end 37.2000 22.8000) (width 0.2500) (layer "F.Cu") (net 7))
 (segment (start 37.2000 22.8000) (end 37.0000 22.6000) (width 0.2500) (layer "F.Cu") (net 7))
 (segment (start 37.0000 22.6000) (end 37.0000 22.2000) (width 0.2500) (layer "F.Cu") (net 7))
 (segment (start 37.0000 22.2000) (end 35.6000 20.8000) (width 0.2500) (layer "F.Cu") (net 7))
 (segment (start 35.6000 20.8000) (end 33.0000 20.8000) (width 0.2500) (layer "F.Cu") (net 7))
 (segment (start 33.0000 20.8000) (end 30.8000 23.0000) (width 0.2500) (layer "F.Cu") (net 7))
 (segment (start 30.8000 23.0000) (end 28.8000 23.0000) (width 0.2500) (layer "F.Cu") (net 7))
 (segment (start 28.8000 21.6000) (end 28.6000 21.6000) (width 0.2500) (layer "F.Cu") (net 8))
 (segment (start 28.6000 21.6000) (end 28.4000 21.4000) (width 0.2500) (layer "F.Cu") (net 8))
 (segment (start 28.4000 21.4000) (end 27.4000 21.4000) (width 0.2500) (layer "F.Cu") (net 8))
 (segment (start 27.4000 21.4000) (end 27.2000 21.2000) (width 0.2500) (layer "F.Cu") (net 8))
 (segment (start 27.2000 21.2000) (end 27.2000 17.2000) (width 0.2500) (layer "F.Cu") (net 8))
 (segment (start 27.2000 17.2000) (end 24.0000 14.0000) (width 0.2500) (layer "F.Cu") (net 8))
 (via (at 12.6000 21.8000) (size 0.6000) (drill 0.3000) (layers "F.Cu" "B.Cu") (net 1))
 (via (at 16.0000 32.0000) (size 0.6000) (drill 0.3000) (layers "F.Cu" "B.Cu") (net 1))
 (via (at 12.6000 24.2000) (size 0.6000) (drill 0.3000) (layers "F.Cu" "B.Cu") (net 1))
 (via (at 24.8000 19.2000) (size 0.6000) (drill 0.3000) (layers "F.Cu" "B.Cu") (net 3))
 (via (at 28.8000 20.4000) (size 0.6000) (drill 0.3000) (layers "F.Cu" "B.Cu") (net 3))
 (via (at 19.4000 21.0000) (size 0.6000) (drill 0.3000) (layers "F.Cu" "B.Cu") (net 3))
 (via (at 22.0000 19.0000) (size 0.6000) (drill 0.3000) (layers "F.Cu" "B.Cu") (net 3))
 (via (at 34.8000 21.8000) (size 0.6000) (drill 0.3000) (layers "F.Cu" "B.Cu") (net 3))
 (via (at 32.8000 20.0000) (size 0.6000) (drill 0.3000) (layers "F.Cu" "B.Cu") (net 3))
 (via (at 37.8000 21.0000) (size 0.6000) (drill 0.3000) (layers "F.Cu" "B.Cu") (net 3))
 (via (at 36.8000 26.2000) (size 0.6000) (drill 0.3000) (layers "F.Cu" "B.Cu") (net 3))
 (via (at 12.6000 23.0000) (size 0.6000) (drill 0.3000) (layers "F.Cu" "B.Cu") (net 2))
 (via (at 35.6000 23.0000) (size 0.6000) (drill 0.3000) (layers "F.Cu" "B.Cu") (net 2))
 (via (at 28.8000 19.0000) (size 0.6000) (drill 0.3000) (layers "F.Cu" "B.Cu") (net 2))
 (via (at 26.2000 18.0000) (size 0.6000) (drill 0.3000) (layers "F.Cu" "B.Cu") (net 2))
 (via (at 32.6000 26.2000) (size 0.6000) (drill 0.3000) (layers "F.Cu" "B.Cu") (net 2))
 (via (at 27.0000 15.2000) (size 0.6000) (drill 0.3000) (layers "F.Cu" "B.Cu") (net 4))
 (via (at 23.2000 20.4000) (size 0.6000) (drill 0.3000) (layers "F.Cu" "B.Cu") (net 4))
 (via (at 33.0000 22.6000) (size 0.6000) (drill 0.3000) (layers "F.Cu" "B.Cu") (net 4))
 (via (at 14.2000 26.4000) (size 0.6000) (drill 0.3000) (layers "F.Cu" "B.Cu") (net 5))
 (via (at 28.6000 25.2000) (size 0.6000) (drill 0.3000) (layers "F.Cu" "B.Cu") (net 5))
 (via (at 23.2000 21.6000) (size 0.6000) (drill 0.3000) (layers "F.Cu" "B.Cu") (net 5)))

